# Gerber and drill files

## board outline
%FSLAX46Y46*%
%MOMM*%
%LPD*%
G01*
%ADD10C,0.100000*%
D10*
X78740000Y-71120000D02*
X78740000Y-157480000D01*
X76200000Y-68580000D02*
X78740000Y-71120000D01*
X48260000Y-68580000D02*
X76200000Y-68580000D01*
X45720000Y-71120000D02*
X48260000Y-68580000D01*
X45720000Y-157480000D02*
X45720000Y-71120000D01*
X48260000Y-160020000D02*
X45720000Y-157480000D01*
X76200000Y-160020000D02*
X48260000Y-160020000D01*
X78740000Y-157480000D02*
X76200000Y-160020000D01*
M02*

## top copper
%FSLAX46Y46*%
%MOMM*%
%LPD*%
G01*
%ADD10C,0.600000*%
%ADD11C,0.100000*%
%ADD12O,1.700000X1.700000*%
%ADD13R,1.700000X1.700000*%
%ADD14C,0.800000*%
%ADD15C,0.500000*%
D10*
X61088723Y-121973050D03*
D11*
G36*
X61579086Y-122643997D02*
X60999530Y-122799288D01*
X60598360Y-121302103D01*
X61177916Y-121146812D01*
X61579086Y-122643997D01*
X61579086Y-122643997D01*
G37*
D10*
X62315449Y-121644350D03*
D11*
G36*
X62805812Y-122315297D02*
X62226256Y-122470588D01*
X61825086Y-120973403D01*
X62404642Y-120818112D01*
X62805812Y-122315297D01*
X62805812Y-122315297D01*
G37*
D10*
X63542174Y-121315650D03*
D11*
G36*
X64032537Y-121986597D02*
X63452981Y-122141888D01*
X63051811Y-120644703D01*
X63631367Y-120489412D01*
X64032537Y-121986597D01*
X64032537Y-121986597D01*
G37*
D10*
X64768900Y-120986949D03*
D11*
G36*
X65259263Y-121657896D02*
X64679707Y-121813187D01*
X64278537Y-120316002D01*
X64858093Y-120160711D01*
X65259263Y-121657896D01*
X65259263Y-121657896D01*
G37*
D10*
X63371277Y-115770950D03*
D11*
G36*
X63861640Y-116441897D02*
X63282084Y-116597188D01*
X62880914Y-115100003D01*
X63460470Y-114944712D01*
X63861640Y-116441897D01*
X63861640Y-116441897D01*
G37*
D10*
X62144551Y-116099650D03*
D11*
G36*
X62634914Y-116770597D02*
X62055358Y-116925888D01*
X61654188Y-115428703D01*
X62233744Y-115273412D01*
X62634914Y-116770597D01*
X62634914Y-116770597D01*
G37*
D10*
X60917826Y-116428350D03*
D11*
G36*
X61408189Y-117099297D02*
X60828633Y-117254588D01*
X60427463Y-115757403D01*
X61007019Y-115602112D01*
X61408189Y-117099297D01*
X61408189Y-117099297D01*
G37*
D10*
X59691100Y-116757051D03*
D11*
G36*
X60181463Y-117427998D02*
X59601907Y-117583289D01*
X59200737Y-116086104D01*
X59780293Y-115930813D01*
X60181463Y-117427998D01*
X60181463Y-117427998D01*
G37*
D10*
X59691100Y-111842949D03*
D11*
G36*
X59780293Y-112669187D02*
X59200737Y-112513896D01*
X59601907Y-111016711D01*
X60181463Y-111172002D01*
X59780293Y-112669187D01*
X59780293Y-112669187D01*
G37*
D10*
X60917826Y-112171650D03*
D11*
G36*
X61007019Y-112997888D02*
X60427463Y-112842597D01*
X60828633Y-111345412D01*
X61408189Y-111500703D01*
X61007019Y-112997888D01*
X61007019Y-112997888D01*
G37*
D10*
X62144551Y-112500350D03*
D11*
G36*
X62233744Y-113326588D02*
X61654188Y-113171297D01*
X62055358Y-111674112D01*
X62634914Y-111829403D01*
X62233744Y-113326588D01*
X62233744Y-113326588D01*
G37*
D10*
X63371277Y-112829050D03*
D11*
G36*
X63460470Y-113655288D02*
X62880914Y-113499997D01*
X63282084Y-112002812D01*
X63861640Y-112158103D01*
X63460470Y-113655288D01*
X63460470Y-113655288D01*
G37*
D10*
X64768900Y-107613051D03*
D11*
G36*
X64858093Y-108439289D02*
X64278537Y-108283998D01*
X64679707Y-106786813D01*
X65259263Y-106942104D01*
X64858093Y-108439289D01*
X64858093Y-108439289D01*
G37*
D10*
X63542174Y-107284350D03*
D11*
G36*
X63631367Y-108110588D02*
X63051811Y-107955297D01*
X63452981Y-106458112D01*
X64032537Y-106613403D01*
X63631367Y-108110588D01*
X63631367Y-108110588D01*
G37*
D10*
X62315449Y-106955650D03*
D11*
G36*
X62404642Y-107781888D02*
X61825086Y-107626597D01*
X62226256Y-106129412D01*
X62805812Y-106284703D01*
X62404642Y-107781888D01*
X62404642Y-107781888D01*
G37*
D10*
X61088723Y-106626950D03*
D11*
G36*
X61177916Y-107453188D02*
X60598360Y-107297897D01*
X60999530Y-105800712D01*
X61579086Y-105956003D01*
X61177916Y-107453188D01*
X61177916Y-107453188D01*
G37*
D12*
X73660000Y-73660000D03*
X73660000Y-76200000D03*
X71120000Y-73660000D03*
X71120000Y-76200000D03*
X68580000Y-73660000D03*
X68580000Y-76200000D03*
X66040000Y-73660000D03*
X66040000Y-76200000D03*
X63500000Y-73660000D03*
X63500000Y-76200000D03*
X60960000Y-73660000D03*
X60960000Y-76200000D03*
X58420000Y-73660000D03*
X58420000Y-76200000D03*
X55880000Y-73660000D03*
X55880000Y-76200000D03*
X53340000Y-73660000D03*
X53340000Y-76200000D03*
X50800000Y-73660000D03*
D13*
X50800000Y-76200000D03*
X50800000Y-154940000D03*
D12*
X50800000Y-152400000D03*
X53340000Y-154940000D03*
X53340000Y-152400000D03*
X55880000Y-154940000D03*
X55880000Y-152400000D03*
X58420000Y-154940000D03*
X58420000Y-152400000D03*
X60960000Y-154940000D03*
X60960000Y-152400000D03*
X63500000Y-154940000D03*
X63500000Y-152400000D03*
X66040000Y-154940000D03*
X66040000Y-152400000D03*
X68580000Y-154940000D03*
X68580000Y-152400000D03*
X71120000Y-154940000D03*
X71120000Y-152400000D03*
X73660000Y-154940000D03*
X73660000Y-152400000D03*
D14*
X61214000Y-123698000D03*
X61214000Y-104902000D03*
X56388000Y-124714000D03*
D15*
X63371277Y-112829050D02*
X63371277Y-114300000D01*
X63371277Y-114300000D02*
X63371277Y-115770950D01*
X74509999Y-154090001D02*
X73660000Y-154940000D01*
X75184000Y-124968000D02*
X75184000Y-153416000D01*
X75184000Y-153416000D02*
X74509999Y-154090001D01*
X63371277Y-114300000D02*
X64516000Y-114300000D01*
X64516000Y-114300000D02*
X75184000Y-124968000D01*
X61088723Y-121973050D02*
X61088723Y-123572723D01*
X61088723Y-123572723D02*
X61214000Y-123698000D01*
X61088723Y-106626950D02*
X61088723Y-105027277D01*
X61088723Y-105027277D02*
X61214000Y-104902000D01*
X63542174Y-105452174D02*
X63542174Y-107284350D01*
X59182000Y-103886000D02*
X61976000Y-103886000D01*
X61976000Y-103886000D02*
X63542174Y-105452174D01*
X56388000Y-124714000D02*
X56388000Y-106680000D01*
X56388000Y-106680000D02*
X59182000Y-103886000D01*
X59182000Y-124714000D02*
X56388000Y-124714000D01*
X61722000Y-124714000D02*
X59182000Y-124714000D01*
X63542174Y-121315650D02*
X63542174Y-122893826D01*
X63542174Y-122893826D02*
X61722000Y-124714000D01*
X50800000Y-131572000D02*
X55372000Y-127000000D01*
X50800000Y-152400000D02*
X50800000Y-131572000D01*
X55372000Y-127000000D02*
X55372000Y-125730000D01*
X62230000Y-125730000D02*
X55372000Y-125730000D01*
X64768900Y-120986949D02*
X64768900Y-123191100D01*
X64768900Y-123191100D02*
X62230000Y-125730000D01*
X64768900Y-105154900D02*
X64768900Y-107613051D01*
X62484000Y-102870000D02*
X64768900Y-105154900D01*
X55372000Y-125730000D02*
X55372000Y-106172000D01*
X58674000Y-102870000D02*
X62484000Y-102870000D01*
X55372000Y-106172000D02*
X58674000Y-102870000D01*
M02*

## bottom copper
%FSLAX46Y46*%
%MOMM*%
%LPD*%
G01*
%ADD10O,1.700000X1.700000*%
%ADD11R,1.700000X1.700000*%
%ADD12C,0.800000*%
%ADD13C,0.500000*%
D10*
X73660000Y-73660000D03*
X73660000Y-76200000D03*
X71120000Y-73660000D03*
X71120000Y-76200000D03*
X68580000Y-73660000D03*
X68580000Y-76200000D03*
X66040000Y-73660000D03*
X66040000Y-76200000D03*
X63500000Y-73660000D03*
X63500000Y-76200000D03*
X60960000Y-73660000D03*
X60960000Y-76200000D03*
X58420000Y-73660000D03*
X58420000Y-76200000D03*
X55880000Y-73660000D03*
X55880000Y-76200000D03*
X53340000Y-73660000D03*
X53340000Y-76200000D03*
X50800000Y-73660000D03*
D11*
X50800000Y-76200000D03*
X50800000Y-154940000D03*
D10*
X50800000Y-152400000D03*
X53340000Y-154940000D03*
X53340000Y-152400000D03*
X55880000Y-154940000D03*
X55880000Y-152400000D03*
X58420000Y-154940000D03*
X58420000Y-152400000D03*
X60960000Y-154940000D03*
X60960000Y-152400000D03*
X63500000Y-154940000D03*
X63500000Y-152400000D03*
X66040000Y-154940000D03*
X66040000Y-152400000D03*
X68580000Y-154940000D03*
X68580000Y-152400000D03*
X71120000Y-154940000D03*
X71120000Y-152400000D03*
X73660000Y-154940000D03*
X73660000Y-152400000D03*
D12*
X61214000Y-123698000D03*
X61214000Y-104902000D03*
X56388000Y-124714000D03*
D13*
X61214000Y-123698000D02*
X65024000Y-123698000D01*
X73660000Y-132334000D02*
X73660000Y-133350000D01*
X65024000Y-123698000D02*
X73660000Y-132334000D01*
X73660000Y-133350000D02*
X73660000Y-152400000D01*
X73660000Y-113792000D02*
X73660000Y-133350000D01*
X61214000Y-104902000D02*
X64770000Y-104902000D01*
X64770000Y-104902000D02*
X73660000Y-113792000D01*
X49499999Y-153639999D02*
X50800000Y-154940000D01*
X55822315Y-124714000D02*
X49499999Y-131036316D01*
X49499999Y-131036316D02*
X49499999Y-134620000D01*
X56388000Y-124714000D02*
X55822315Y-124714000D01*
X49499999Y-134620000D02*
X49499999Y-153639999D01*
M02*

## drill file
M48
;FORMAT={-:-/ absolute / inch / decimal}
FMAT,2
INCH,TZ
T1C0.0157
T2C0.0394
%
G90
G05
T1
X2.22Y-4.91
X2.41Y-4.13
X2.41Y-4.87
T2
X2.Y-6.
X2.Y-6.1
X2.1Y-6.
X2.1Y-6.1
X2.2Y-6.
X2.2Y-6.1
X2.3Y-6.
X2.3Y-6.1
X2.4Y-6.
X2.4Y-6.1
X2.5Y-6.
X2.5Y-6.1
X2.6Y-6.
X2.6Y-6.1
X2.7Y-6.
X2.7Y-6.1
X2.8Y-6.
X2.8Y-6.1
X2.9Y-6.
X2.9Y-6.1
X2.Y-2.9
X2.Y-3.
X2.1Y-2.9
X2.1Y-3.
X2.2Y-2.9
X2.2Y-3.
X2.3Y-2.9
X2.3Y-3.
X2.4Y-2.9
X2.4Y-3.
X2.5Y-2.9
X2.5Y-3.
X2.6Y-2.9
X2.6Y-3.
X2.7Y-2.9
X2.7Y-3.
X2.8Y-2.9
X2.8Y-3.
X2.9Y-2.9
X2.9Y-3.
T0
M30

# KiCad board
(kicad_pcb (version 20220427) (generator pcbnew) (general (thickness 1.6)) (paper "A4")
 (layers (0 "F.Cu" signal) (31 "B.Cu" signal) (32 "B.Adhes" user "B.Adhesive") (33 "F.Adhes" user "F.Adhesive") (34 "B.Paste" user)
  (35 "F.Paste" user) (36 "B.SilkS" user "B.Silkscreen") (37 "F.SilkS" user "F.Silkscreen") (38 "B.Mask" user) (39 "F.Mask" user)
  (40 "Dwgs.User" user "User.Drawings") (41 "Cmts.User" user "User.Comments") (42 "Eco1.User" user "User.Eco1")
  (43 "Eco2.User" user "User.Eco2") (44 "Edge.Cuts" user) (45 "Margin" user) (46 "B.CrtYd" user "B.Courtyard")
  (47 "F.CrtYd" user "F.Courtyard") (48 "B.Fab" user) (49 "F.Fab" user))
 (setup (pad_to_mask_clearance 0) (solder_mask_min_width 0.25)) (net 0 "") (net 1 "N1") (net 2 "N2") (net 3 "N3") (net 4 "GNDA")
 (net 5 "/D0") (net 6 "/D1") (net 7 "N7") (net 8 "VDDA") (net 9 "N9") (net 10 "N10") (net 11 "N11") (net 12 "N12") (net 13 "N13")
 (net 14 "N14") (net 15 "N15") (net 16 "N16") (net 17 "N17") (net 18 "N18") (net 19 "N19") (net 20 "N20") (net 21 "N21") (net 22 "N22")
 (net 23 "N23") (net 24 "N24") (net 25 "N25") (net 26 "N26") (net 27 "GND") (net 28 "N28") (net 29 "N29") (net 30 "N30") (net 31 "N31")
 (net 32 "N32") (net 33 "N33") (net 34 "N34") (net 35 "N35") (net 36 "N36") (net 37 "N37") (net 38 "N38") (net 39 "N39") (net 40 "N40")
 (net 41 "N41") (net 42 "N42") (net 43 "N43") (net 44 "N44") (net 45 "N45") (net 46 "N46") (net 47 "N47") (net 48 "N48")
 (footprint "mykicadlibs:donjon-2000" (layer "F.Cu") (at 62.23 85.725)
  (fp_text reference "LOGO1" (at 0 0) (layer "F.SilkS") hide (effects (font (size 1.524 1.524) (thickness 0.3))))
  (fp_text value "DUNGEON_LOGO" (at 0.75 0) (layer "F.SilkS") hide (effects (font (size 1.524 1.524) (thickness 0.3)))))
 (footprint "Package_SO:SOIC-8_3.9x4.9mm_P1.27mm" (layer "F.Cu") (at 62.23 109.728 75)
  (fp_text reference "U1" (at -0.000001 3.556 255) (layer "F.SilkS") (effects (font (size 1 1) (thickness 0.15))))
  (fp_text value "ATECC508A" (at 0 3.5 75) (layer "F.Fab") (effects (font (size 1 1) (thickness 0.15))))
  (pad "1" smd rect locked (at -2.7 -1.905 75) (size 1.55 0.6) (layers "F.Cu" "F.Paste" "F.Mask") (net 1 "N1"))
  (pad "2" smd rect locked (at -2.7 -0.635 75) (size 1.55 0.6) (layers "F.Cu" "F.Paste" "F.Mask") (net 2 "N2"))
  (pad "3" smd rect locked (at -2.7 0.635 75) (size 1.55 0.6) (layers "F.Cu" "F.Paste" "F.Mask") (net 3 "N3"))
  (pad "4" smd rect locked (at -2.7 1.905 75) (size 1.55 0.6) (layers "F.Cu" "F.Paste" "F.Mask") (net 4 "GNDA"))
  (pad "5" smd rect locked (at 2.7 1.905 75) (size 1.55 0.6) (layers "F.Cu" "F.Paste" "F.Mask") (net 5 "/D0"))
  (pad "6" smd rect locked (at 2.7 0.635 75) (size 1.55 0.6) (layers "F.Cu" "F.Paste" "F.Mask") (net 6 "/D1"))
  (pad "7" smd rect locked (at 2.7 -0.635 75) (size 1.55 0.6) (layers "F.Cu" "F.Paste" "F.Mask") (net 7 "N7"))
  (pad "8" smd rect locked (at 2.7 -1.905 75) (size 1.55 0.6) (layers "F.Cu" "F.Paste" "F.Mask") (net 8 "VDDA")))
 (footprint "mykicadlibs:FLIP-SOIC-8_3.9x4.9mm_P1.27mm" (layer "F.Cu") (at 62.23 118.872 105)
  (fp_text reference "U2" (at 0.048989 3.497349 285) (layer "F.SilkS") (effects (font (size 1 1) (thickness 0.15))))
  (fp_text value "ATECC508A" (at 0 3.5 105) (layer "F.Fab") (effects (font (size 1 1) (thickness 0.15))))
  (pad "1" smd rect locked (at 2.7 -1.905 105) (size 1.55 0.6) (layers "F.Cu" "F.Paste" "F.Mask") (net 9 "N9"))
  (pad "2" smd rect locked (at 2.7 -0.635 105) (size 1.55 0.6) (layers "F.Cu" "F.Paste" "F.Mask") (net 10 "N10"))
  (pad "3" smd rect locked (at 2.7 0.635 105) (size 1.55 0.6) (layers "F.Cu" "F.Paste" "F.Mask") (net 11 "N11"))
  (pad "4" smd rect locked (at 2.7 1.905 105) (size 1.55 0.6) (layers "F.Cu" "F.Paste" "F.Mask") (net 4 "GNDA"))
  (pad "5" smd rect locked (at -2.7 1.905 105) (size 1.55 0.6) (layers "F.Cu" "F.Paste" "F.Mask") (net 5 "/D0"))
  (pad "6" smd rect locked (at -2.7 0.635 105) (size 1.55 0.6) (layers "F.Cu" "F.Paste" "F.Mask") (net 6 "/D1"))
  (pad "7" smd rect locked (at -2.7 -0.635 105) (size 1.55 0.6) (layers "F.Cu" "F.Paste" "F.Mask") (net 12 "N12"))
  (pad "8" smd rect locked (at -2.7 -1.905 105) (size 1.55 0.6) (layers "F.Cu" "F.Paste" "F.Mask") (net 8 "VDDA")))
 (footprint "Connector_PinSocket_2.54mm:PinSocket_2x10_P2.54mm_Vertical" (layer "B.Cu") (at 50.8 154.94 -90)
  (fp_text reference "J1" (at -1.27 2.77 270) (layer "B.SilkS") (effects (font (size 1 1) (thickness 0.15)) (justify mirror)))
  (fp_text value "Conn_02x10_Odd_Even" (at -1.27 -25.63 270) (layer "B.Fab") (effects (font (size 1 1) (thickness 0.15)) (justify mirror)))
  (pad "1" thru_hole rect locked (at 0 0 270) (size 1.7 1.7) (drill 1) (layers *.Cu *.Mask) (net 6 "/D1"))
  (pad "2" thru_hole oval locked (at -2.54 0 270) (size 1.7 1.7) (drill 1) (layers *.Cu *.Mask) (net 5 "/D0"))
  (pad "3" thru_hole oval locked (at 0 -2.54 270) (size 1.7 1.7) (drill 1) (layers *.Cu *.Mask) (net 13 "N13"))
  (pad "4" thru_hole oval locked (at -2.54 -2.54 270) (size 1.7 1.7) (drill 1) (layers *.Cu *.Mask) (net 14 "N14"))
  (pad "5" thru_hole oval locked (at 0 -5.08 270) (size 1.7 1.7) (drill 1) (layers *.Cu *.Mask) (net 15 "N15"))
  (pad "6" thru_hole oval locked (at -2.54 -5.08 270) (size 1.7 1.7) (drill 1) (layers *.Cu *.Mask) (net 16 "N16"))
  (pad "7" thru_hole oval locked (at 0 -7.62 270) (size 1.7 1.7) (drill 1) (layers *.Cu *.Mask) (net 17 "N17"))
  (pad "8" thru_hole oval locked (at -2.54 -7.62 270) (size 1.7 1.7) (drill 1) (layers *.Cu *.Mask) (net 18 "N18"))
  (pad "9" thru_hole oval locked (at 0 -10.16 270) (size 1.7 1.7) (drill 1) (layers *.Cu *.Mask) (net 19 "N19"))
  (pad "10" thru_hole oval locked (at -2.54 -10.16 270) (size 1.7 1.7) (drill 1) (layers *.Cu *.Mask) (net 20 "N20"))
  (pad "11" thru_hole oval locked (at 0 -12.7 270) (size 1.7 1.7) (drill 1) (layers *.Cu *.Mask) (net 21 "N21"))
  (pad "12" thru_hole oval locked (at -2.54 -12.7 270) (size 1.7 1.7) (drill 1) (layers *.Cu *.Mask) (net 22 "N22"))
  (pad "13" thru_hole oval locked (at 0 -15.24 270) (size 1.7 1.7) (drill 1) (layers *.Cu *.Mask) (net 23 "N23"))
  (pad "14" thru_hole oval locked (at -2.54 -15.24 270) (size 1.7 1.7) (drill 1) (layers *.Cu *.Mask) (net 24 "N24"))
  (pad "15" thru_hole oval locked (at 0 -17.78 270) (size 1.7 1.7) (drill 1) (layers *.Cu *.Mask) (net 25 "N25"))
  (pad "16" thru_hole oval locked (at -2.54 -17.78 270) (size 1.7 1.7) (drill 1) (layers *.Cu *.Mask) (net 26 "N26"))
  (pad "17" thru_hole oval locked (at 0 -20.32 270) (size 1.7 1.7) (drill 1) (layers *.Cu *.Mask) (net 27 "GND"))
  (pad "18" thru_hole oval locked (at -2.54 -20.32 270) (size 1.7 1.7) (drill 1) (layers *.Cu *.Mask) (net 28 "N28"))
  (pad "19" thru_hole oval locked (at 0 -22.86 270) (size 1.7 1.7) (drill 1) (layers *.Cu *.Mask) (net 4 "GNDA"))
  (pad "20" thru_hole oval locked (at -2.54 -22.86 270) (size 1.7 1.7) (drill 1) (layers *.Cu *.Mask) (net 8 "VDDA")))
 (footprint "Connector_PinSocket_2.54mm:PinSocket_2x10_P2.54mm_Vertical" (layer "B.Cu") (at 50.8 76.2 -90)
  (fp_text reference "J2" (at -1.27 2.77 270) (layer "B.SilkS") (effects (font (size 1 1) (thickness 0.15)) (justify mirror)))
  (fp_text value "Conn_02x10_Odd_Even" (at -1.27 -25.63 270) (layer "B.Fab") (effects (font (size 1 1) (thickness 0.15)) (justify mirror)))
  (pad "1" thru_hole rect locked (at 0 0 270) (size 1.7 1.7) (drill 1) (layers *.Cu *.Mask) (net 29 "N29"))
  (pad "2" thru_hole oval locked (at -2.54 0 270) (size 1.7 1.7) (drill 1) (layers *.Cu *.Mask) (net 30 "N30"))
  (pad "3" thru_hole oval locked (at 0 -2.54 270) (size 1.7 1.7) (drill 1) (layers *.Cu *.Mask) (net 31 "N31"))
  (pad "4" thru_hole oval locked (at -2.54 -2.54 270) (size 1.7 1.7) (drill 1) (layers *.Cu *.Mask) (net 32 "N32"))
  (pad "5" thru_hole oval locked (at 0 -5.08 270) (size 1.7 1.7) (drill 1) (layers *.Cu *.Mask) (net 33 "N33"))
  (pad "6" thru_hole oval locked (at -2.54 -5.08 270) (size 1.7 1.7) (drill 1) (layers *.Cu *.Mask) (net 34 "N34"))
  (pad "7" thru_hole oval locked (at 0 -7.62 270) (size 1.7 1.7) (drill 1) (layers *.Cu *.Mask) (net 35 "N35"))
  (pad "8" thru_hole oval locked (at -2.54 -7.62 270) (size 1.7 1.7) (drill 1) (layers *.Cu *.Mask) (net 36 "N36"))
  (pad "9" thru_hole oval locked (at 0 -10.16 270) (size 1.7 1.7) (drill 1) (layers *.Cu *.Mask) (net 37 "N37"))
  (pad "10" thru_hole oval locked (at -2.54 -10.16 270) (size 1.7 1.7) (drill 1) (layers *.Cu *.Mask) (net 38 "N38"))
  (pad "11" thru_hole oval locked (at 0 -12.7 270) (size 1.7 1.7) (drill 1) (layers *.Cu *.Mask) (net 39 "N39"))
  (pad "12" thru_hole oval locked (at -2.54 -12.7 270) (size 1.7 1.7) (drill 1) (layers *.Cu *.Mask) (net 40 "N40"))
  (pad "13" thru_hole oval locked (at 0 -15.24 270) (size 1.7 1.7) (drill 1) (layers *.Cu *.Mask) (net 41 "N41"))
  (pad "14" thru_hole oval locked (at -2.54 -15.24 270) (size 1.7 1.7) (drill 1) (layers *.Cu *.Mask) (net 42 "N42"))
  (pad "15" thru_hole oval locked (at 0 -17.78 270) (size 1.7 1.7) (drill 1) (layers *.Cu *.Mask) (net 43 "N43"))
  (pad "16" thru_hole oval locked (at -2.54 -17.78 270) (size 1.7 1.7) (drill 1) (layers *.Cu *.Mask) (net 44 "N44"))
  (pad "17" thru_hole oval locked (at 0 -20.32 270) (size 1.7 1.7) (drill 1) (layers *.Cu *.Mask) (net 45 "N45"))
  (pad "18" thru_hole oval locked (at -2.54 -20.32 270) (size 1.7 1.7) (drill 1) (layers *.Cu *.Mask) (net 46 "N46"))
  (pad "19" thru_hole oval locked (at 0 -22.86 270) (size 1.7 1.7) (drill 1) (layers *.Cu *.Mask) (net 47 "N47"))
  (pad "20" thru_hole oval locked (at -2.54 -22.86 270) (size 1.7 1.7) (drill 1) (layers *.Cu *.Mask) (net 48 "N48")))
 (gr_line (start 48.26 68.58) (end 76.2 68.58) (stroke (width 0.1) (type solid)) (layer "Edge.Cuts"))
 (gr_line (start 76.2 68.58) (end 78.74 71.12) (stroke (width 0.1) (type solid)) (layer "Edge.Cuts"))
 (gr_line (start 48.26 160.02) (end 45.72 157.48) (stroke (width 0.1) (type solid)) (layer "Edge.Cuts"))
 (gr_line (start 78.74 71.12) (end 78.74 157.48) (stroke (width 0.1) (type solid)) (layer "Edge.Cuts"))
 (gr_line (start 45.72 157.48) (end 45.72 71.12) (stroke (width 0.1) (type solid)) (layer "Edge.Cuts"))
 (gr_line (start 78.74 157.48) (end 76.2 160.02) (stroke (width 0.1) (type solid)) (layer "Edge.Cuts"))
 (gr_line (start 76.2 160.02) (end 48.26 160.02) (stroke (width 0.1) (type solid)) (layer "Edge.Cuts"))
 (gr_line (start 45.72 71.12) (end 48.26 68.58) (stroke (width 0.1) (type solid)) (layer "Edge.Cuts"))
 (segment (start 64.516 114.3) (end 75.184 124.968) (width 0.5) (layer "F.Cu") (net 4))
 (segment (start 63.371277 114.3) (end 64.516 114.3) (width 0.5) (layer "F.Cu") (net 4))
 (segment (start 74.509999 154.090001) (end 73.66 154.94) (width 0.5) (layer "F.Cu") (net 4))
 (segment (start 75.184 124.968) (end 75.184 153.416) (width 0.5) (layer "F.Cu") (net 4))
 (segment (start 63.371277 114.3) (end 63.371277 115.77095) (width 0.5) (layer "F.Cu") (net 4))
 (segment (start 75.184 153.416) (end 74.509999 154.090001) (width 0.5) (layer "F.Cu") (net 4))
 (segment (start 63.371277 112.82905) (end 63.371277 114.3) (width 0.5) (layer "F.Cu") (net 4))
 (segment (start 61.088723 121.97305) (end 61.088723 123.572723) (width 0.5) (layer "F.Cu") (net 8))
 (segment (start 61.088723 106.62695) (end 61.088723 105.027277) (width 0.5) (layer "F.Cu") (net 8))
 (segment (start 61.088723 105.027277) (end 61.214 104.902) (width 0.5) (layer "F.Cu") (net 8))
 (segment (start 61.088723 123.572723) (end 61.214 123.698) (width 0.5) (layer "F.Cu") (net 8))
 (via (at 61.214 104.902) (size 0.8) (drill 0.4) (layers "F.Cu" "B.Cu") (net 8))
 (via (at 61.214 123.698) (size 0.8) (drill 0.4) (layers "F.Cu" "B.Cu") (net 8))
 (segment (start 73.66 132.334) (end 73.66 133.35) (width 0.5) (layer "B.Cu") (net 8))
 (segment (start 73.66 133.35) (end 73.66 152.4) (width 0.5) (layer "B.Cu") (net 8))
 (segment (start 64.77 104.902) (end 73.66 113.792) (width 0.5) (layer "B.Cu") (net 8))
 (segment (start 61.214 123.698) (end 65.024 123.698) (width 0.5) (layer "B.Cu") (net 8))
 (segment (start 65.024 123.698) (end 73.66 132.334) (width 0.5) (layer "B.Cu") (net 8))
 (segment (start 73.66 113.792) (end 73.66 133.35) (width 0.5) (layer "B.Cu") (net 8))
 (segment (start 61.214 104.902) (end 64.77 104.902) (width 0.5) (layer "B.Cu") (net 8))
 (segment (start 63.542174 122.893826) (end 61.722 124.714) (width 0.5) (layer "F.Cu") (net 6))
 (segment (start 56.388 106.68) (end 59.182 103.886) (width 0.5) (layer "F.Cu") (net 6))
 (segment (start 56.388 124.714) (end 56.388 106.68) (width 0.5) (layer "F.Cu") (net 6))
 (segment (start 59.182 124.714) (end 56.388 124.714) (width 0.5) (layer "F.Cu") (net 6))
 (segment (start 59.182 103.886) (end 61.976 103.886) (width 0.5) (layer "F.Cu") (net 6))
 (segment (start 61.722 124.714) (end 59.182 124.714) (width 0.5) (layer "F.Cu") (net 6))
 (segment (start 63.542174 121.31565) (end 63.542174 122.893826) (width 0.5) (layer "F.Cu") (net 6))
 (segment (start 61.976 103.886) (end 63.542174 105.452174) (width 0.5) (layer "F.Cu") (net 6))
 (segment (start 63.542174 105.452174) (end 63.542174 107.28435) (width 0.5) (layer "F.Cu") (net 6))
 (via (at 56.388 124.714) (size 0.8) (drill 0.4) (layers "F.Cu" "B.Cu") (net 6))
 (segment (start 49.499999 153.639999) (end 50.8 154.94) (width 0.5) (layer "B.Cu") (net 6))
 (segment (start 49.499999 131.036316) (end 49.499999 134.62) (width 0.5) (layer "B.Cu") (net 6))
 (segment (start 55.822315 124.714) (end 49.499999 131.036316) (width 0.5) (layer "B.Cu") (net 6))
 (segment (start 56.388 124.714) (end 55.822315 124.714) (width 0.5) (layer "B.Cu") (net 6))
 (segment (start 49.499999 134.62) (end 49.499999 153.639999) (width 0.5) (layer "B.Cu") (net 6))
 (segment (start 58.674 102.87) (end 62.484 102.87) (width 0.5) (layer "F.Cu") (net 5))
 (segment (start 64.7689 120.986949) (end 64.7689 123.1911) (width 0.5) (layer "F.Cu") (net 5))
 (segment (start 55.372 106.172) (end 58.674 102.87) (width 0.5) (layer "F.Cu") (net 5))
 (segment (start 64.7689 123.1911) (end 62.23 125.73) (width 0.5) (layer "F.Cu") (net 5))
 (segment (start 50.8 152.4) (end 50.8 131.572) (width 0.5) (layer "F.Cu") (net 5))
 (segment (start 50.8 131.572) (end 55.372 127) (width 0.5) (layer "F.Cu") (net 5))
 (segment (start 55.372 127) (end 55.372 125.73) (width 0.5) (layer "F.Cu") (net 5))
 (segment (start 62.23 125.73) (end 55.372 125.73) (width 0.5) (layer "F.Cu") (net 5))
 (segment (start 62.484 102.87) (end 64.7689 105.1549) (width 0.5) (layer "F.Cu") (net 5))
 (segment (start 55.372 125.73) (end 55.372 106.172) (width 0.5) (layer "F.Cu") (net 5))
 (segment (start 64.7689 105.1549) (end 64.7689 107.613051) (width 0.5) (layer "F.Cu") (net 5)))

